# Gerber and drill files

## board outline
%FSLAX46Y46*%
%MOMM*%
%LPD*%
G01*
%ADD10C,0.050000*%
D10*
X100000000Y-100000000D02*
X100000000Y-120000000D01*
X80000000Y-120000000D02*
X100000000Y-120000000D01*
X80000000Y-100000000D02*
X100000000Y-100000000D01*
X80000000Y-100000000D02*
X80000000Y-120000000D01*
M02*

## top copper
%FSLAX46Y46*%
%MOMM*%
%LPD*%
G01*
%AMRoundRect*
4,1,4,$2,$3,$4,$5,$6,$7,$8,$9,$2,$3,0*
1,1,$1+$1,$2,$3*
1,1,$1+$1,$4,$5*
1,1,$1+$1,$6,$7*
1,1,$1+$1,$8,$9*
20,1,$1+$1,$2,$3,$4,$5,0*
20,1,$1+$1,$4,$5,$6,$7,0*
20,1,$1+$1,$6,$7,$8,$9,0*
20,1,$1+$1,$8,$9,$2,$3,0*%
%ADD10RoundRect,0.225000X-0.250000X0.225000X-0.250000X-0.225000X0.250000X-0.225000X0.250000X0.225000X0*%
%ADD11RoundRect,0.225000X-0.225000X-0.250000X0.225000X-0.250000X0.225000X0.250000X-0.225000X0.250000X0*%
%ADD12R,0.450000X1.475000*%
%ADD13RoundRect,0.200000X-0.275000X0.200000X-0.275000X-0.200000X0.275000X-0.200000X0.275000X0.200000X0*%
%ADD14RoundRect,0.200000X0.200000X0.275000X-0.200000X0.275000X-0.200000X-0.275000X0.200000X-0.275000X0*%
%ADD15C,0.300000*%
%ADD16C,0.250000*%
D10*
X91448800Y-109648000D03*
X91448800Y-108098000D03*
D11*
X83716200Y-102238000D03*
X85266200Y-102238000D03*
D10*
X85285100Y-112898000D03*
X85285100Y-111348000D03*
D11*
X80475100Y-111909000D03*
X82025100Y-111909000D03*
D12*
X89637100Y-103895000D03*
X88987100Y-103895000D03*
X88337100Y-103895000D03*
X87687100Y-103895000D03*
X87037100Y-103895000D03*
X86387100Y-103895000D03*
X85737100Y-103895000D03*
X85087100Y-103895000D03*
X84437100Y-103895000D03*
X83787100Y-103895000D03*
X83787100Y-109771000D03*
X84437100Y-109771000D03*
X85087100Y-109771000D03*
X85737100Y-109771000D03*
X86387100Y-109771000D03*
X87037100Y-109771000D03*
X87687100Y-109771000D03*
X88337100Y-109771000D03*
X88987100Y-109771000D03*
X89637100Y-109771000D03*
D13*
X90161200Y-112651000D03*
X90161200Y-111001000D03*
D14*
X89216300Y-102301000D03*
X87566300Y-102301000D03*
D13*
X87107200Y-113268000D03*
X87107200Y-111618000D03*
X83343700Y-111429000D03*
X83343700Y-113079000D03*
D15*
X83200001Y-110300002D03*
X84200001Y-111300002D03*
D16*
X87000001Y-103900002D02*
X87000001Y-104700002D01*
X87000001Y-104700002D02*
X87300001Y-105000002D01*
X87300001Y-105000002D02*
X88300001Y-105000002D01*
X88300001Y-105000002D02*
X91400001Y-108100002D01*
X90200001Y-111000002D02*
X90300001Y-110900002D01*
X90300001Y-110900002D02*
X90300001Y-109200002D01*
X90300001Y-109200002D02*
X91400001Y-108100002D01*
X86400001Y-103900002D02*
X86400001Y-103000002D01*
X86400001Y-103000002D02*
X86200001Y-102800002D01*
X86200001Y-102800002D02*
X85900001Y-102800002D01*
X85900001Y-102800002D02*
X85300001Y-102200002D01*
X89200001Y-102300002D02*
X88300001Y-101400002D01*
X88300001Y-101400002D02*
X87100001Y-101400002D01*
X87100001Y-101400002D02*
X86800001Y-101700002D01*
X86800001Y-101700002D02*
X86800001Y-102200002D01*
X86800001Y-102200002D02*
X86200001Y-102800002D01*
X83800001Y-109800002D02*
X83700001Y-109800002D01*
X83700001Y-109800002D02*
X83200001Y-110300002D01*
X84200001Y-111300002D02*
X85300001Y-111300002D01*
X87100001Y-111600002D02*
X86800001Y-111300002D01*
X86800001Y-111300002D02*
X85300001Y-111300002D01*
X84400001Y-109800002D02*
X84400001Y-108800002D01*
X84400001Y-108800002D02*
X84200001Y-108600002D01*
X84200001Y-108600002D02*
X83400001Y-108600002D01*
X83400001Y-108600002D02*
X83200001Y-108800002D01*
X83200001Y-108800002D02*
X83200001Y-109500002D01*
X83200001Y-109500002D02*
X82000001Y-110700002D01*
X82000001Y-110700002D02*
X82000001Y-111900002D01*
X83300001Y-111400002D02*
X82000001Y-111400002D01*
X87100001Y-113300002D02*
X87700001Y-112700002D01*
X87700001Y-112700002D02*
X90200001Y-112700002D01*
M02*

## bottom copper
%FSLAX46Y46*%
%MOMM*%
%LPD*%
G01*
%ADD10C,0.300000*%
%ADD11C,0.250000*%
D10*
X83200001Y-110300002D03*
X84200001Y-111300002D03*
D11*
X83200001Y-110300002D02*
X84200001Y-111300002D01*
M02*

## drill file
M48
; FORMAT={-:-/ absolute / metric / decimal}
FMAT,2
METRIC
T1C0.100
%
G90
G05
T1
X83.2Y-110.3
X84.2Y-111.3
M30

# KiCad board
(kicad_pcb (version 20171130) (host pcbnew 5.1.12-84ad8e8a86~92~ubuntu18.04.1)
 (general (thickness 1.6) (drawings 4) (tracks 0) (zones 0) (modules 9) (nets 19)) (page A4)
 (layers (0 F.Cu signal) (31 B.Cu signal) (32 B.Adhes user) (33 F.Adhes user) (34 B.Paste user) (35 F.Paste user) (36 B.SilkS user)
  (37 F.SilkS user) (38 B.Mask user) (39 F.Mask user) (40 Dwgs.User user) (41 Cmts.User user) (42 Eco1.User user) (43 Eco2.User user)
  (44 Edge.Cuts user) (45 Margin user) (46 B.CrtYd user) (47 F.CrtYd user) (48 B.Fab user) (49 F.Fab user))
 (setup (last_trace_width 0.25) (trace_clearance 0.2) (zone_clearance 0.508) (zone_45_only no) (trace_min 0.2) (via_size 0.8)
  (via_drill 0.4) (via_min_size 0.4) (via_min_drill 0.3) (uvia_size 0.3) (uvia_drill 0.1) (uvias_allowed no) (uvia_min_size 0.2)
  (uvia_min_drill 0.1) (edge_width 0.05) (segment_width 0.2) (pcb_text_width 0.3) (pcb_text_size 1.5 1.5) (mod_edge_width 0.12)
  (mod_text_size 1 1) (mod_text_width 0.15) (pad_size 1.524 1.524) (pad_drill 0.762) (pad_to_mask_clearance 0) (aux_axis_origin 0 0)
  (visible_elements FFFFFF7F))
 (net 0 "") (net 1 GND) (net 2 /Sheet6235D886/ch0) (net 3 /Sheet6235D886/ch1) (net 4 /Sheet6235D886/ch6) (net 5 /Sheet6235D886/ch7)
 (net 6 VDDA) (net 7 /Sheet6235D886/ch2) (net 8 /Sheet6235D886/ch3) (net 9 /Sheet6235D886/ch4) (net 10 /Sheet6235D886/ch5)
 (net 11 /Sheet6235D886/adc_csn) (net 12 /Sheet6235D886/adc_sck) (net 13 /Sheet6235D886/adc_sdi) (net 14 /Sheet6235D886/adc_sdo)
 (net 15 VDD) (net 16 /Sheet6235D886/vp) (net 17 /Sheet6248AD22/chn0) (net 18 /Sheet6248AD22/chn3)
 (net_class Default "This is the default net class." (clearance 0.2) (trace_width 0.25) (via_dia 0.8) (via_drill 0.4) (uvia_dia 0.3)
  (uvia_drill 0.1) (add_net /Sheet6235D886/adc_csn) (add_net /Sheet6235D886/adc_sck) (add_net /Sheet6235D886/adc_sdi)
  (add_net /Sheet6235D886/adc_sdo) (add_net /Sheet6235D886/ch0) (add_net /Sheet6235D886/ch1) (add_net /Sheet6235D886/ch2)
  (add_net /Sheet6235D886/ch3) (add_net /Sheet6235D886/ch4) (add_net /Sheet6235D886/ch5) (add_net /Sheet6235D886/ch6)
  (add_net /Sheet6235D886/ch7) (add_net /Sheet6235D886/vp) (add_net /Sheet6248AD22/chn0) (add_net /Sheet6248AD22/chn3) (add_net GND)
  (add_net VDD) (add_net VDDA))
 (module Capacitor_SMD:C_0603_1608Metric (layer F.Cu) (at 91.448800 108.873000 270.000000)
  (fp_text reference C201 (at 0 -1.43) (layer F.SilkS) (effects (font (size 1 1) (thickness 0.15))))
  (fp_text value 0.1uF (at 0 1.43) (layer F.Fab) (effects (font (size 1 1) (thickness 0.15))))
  (pad 2 smd roundrect (at 0.775 0 270.000000) (size 0.9 0.95) (layers F.Cu F.Mask F.Paste) (roundrect_rratio 0.25) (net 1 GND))
  (pad 1 smd roundrect (at -0.775 0 270.000000) (size 0.9 0.95) (layers F.Cu F.Mask F.Paste) (roundrect_rratio 0.25)
   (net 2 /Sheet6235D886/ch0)))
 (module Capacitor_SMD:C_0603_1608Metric (layer F.Cu) (at 84.491200 102.238000)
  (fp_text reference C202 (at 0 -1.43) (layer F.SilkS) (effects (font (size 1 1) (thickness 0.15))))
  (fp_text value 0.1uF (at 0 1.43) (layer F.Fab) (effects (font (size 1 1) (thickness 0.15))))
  (pad 1 smd roundrect (at -0.775 0) (size 0.9 0.95) (layers F.Cu F.Mask F.Paste) (roundrect_rratio 0.25) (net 1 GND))
  (pad 2 smd roundrect (at 0.775 0) (size 0.9 0.95) (layers F.Cu F.Mask F.Paste) (roundrect_rratio 0.25) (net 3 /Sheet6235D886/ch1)))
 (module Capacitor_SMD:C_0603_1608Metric (layer F.Cu) (at 85.285100 112.123000 270.000000)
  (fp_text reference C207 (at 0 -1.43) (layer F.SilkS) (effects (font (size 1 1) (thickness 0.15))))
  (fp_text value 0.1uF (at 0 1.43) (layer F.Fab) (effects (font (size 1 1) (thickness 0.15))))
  (pad 2 smd roundrect (at 0.775 0 270.000000) (size 0.9 0.95) (layers F.Cu F.Mask F.Paste) (roundrect_rratio 0.25) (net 1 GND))
  (pad 1 smd roundrect (at -0.775 0 270.000000) (size 0.9 0.95) (layers F.Cu F.Mask F.Paste) (roundrect_rratio 0.25)
   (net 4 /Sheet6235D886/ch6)))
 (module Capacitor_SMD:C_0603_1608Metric (layer F.Cu) (at 81.250100 111.909000)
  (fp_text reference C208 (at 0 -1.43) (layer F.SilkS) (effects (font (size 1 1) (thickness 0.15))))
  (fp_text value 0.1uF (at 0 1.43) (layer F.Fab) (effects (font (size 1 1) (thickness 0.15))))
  (pad 1 smd roundrect (at -0.775 0) (size 0.9 0.95) (layers F.Cu F.Mask F.Paste) (roundrect_rratio 0.25) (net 1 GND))
  (pad 2 smd roundrect (at 0.775 0) (size 0.9 0.95) (layers F.Cu F.Mask F.Paste) (roundrect_rratio 0.25) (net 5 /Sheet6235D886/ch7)))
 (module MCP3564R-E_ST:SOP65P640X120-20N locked (layer F.Cu) (at 86.712100 106.833000 270.000000)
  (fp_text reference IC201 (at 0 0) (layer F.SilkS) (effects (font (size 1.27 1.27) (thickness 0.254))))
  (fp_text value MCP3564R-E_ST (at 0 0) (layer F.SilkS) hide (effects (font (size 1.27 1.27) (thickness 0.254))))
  (pad 1 smd rect (at -2.938 -2.925) (size 0.45 1.475) (layers F.Cu F.Mask F.Paste) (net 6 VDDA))
  (pad 2 smd rect (at -2.938 -2.275) (size 0.45 1.475) (layers F.Cu F.Mask F.Paste) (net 1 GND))
  (pad 3 smd rect (at -2.938 -1.625) (size 0.45 1.475) (layers F.Cu F.Mask F.Paste) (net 1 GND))
  (pad 4 smd rect (at -2.938 -0.975) (size 0.45 1.475) (layers F.Cu F.Mask F.Paste))
  (pad 5 smd rect (at -2.938 -0.325) (size 0.45 1.475) (layers F.Cu F.Mask F.Paste) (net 2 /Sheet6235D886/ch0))
  (pad 6 smd rect (at -2.938 0.325) (size 0.45 1.475) (layers F.Cu F.Mask F.Paste) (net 3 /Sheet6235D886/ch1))
  (pad 7 smd rect (at -2.938 0.975) (size 0.45 1.475) (layers F.Cu F.Mask F.Paste) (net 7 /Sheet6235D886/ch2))
  (pad 8 smd rect (at -2.938 1.625) (size 0.45 1.475) (layers F.Cu F.Mask F.Paste) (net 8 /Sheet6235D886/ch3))
  (pad 9 smd rect (at -2.938 2.275) (size 0.45 1.475) (layers F.Cu F.Mask F.Paste) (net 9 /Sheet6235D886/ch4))
  (pad 10 smd rect (at -2.938 2.925) (size 0.45 1.475) (layers F.Cu F.Mask F.Paste) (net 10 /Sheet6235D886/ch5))
  (pad 11 smd rect (at 2.938 2.925) (size 0.45 1.475) (layers F.Cu F.Mask F.Paste) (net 4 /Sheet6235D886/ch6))
  (pad 12 smd rect (at 2.938 2.275) (size 0.45 1.475) (layers F.Cu F.Mask F.Paste) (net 5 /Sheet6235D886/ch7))
  (pad 13 smd rect (at 2.938 1.625) (size 0.45 1.475) (layers F.Cu F.Mask F.Paste) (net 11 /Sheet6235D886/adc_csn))
  (pad 14 smd rect (at 2.938 0.975) (size 0.45 1.475) (layers F.Cu F.Mask F.Paste) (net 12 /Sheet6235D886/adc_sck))
  (pad 15 smd rect (at 2.938 0.325) (size 0.45 1.475) (layers F.Cu F.Mask F.Paste) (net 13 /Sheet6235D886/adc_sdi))
  (pad 16 smd rect (at 2.938 -0.325) (size 0.45 1.475) (layers F.Cu F.Mask F.Paste) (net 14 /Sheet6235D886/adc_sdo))
  (pad 17 smd rect (at 2.938 -0.975) (size 0.45 1.475) (layers F.Cu F.Mask F.Paste))
  (pad 18 smd rect (at 2.938 -1.625) (size 0.45 1.475) (layers F.Cu F.Mask F.Paste))
  (pad 19 smd rect (at 2.938 -2.275) (size 0.45 1.475) (layers F.Cu F.Mask F.Paste) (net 1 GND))
  (pad 20 smd rect (at 2.938 -2.925) (size 0.45 1.475) (layers F.Cu F.Mask F.Paste) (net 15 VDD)))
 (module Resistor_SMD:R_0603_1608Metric (layer F.Cu) (at 90.161200 111.826000 270.000000)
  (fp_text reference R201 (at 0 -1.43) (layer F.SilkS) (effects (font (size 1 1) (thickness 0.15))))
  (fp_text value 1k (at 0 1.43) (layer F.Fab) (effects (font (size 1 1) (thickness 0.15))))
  (pad 2 smd roundrect (at 0.825 0 270.000000) (size 0.8 0.95) (layers F.Cu F.Mask F.Paste) (roundrect_rratio 0.25)
   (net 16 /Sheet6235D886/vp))
  (pad 1 smd roundrect (at -0.825 0 270.000000) (size 0.8 0.95) (layers F.Cu F.Mask F.Paste) (roundrect_rratio 0.25)
   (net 2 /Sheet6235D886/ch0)))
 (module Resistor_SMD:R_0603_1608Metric (layer F.Cu) (at 88.391300 102.301000 180.000000)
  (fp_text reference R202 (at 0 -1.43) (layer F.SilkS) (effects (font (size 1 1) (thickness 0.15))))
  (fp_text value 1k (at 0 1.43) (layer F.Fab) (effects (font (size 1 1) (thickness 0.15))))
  (pad 1 smd roundrect (at -0.825 0 180.000000) (size 0.8 0.95) (layers F.Cu F.Mask F.Paste) (roundrect_rratio 0.25)
   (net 3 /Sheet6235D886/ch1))
  (pad 2 smd roundrect (at 0.825 0 180.000000) (size 0.8 0.95) (layers F.Cu F.Mask F.Paste) (roundrect_rratio 0.25)
   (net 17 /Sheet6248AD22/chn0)))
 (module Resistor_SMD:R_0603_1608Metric (layer F.Cu) (at 87.107200 112.443000 270.000000)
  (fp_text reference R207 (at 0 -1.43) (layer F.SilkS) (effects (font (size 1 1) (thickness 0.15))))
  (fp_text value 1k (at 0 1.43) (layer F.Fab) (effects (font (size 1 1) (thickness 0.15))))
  (pad 2 smd roundrect (at 0.825 0 270.000000) (size 0.8 0.95) (layers F.Cu F.Mask F.Paste) (roundrect_rratio 0.25)
   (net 16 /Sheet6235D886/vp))
  (pad 1 smd roundrect (at -0.825 0 270.000000) (size 0.8 0.95) (layers F.Cu F.Mask F.Paste) (roundrect_rratio 0.25)
   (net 4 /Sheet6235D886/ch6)))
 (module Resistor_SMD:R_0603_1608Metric (layer F.Cu) (at 83.343700 112.254000 270.000000)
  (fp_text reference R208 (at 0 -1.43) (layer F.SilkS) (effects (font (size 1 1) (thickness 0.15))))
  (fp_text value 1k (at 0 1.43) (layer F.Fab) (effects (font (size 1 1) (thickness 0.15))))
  (pad 1 smd roundrect (at -0.825 0 270.000000) (size 0.8 0.95) (layers F.Cu F.Mask F.Paste) (roundrect_rratio 0.25)
   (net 5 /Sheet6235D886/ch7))
  (pad 2 smd roundrect (at 0.825 0 270.000000) (size 0.8 0.95) (layers F.Cu F.Mask F.Paste) (roundrect_rratio 0.25)
   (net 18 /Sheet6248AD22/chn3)))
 (gr_line (start 100 100) (end 100 120) (layer Edge.Cuts) (width 0.05))
 (gr_line (start 80 120) (end 100 120) (layer Edge.Cuts) (width 0.05))
 (gr_line (start 80 100) (end 100 100) (layer Edge.Cuts) (width 0.05))
 (gr_line (start 80 100) (end 80 120) (layer Edge.Cuts) (width 0.05))
 (segment (start 87.000001 103.900002) (end 87.000001 104.700002) (width 0.250000) (layer F.Cu) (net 2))
 (segment (start 87.000001 104.700002) (end 87.300001 105.000002) (width 0.250000) (layer F.Cu) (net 2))
 (segment (start 87.300001 105.000002) (end 88.300001 105.000002) (width 0.250000) (layer F.Cu) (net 2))
 (segment (start 88.300001 105.000002) (end 91.400001 108.100002) (width 0.250000) (layer F.Cu) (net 2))
 (segment (start 90.200001 111.000002) (end 90.300001 110.900002) (width 0.250000) (layer F.Cu) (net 2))
 (segment (start 90.300001 110.900002) (end 90.300001 109.200002) (width 0.250000) (layer F.Cu) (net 2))
 (segment (start 90.300001 109.200002) (end 91.400001 108.100002) (width 0.250000) (layer F.Cu) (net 2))
 (segment (start 86.400001 103.900002) (end 86.400001 103.000002) (width 0.250000) (layer F.Cu) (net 3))
 (segment (start 86.400001 103.000002) (end 86.200001 102.800002) (width 0.250000) (layer F.Cu) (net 3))
 (segment (start 86.200001 102.800002) (end 85.900001 102.800002) (width 0.250000) (layer F.Cu) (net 3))
 (segment (start 85.900001 102.800002) (end 85.300001 102.200002) (width 0.250000) (layer F.Cu) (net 3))
 (segment (start 89.200001 102.300002) (end 88.300001 101.400002) (width 0.250000) (layer F.Cu) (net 3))
 (segment (start 88.300001 101.400002) (end 87.100001 101.400002) (width 0.250000) (layer F.Cu) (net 3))
 (segment (start 87.100001 101.400002) (end 86.800001 101.700002) (width 0.250000) (layer F.Cu) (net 3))
 (segment (start 86.800001 101.700002) (end 86.800001 102.200002) (width 0.250000) (layer F.Cu) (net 3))
 (segment (start 86.800001 102.200002) (end 86.200001 102.800002) (width 0.250000) (layer F.Cu) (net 3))
 (segment (start 83.800001 109.800002) (end 83.700001 109.800002) (width 0.250000) (layer F.Cu) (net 4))
 (segment (start 83.700001 109.800002) (end 83.200001 110.300002) (width 0.250000) (layer F.Cu) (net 4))
 (segment (start 83.200001 110.300002) (end 84.200001 111.300002) (width 0.250000) (layer B.Cu) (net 4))
 (segment (start 84.200001 111.300002) (end 85.300001 111.300002) (width 0.250000) (layer F.Cu) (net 4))
 (segment (start 87.100001 111.600002) (end 86.800001 111.300002) (width 0.250000) (layer F.Cu) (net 4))
 (segment (start 86.800001 111.300002) (end 85.300001 111.300002) (width 0.250000) (layer F.Cu) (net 4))
 (via micro (at 83.200001 110.300002) (size 0.300000) (drill 0.100000) (layers F.Cu B.Cu) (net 4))
 (via micro (at 84.200001 111.300002) (size 0.300000) (drill 0.100000) (layers F.Cu B.Cu) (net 4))
 (segment (start 84.400001 109.800002) (end 84.400001 108.800002) (width 0.250000) (layer F.Cu) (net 5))
 (segment (start 84.400001 108.800002) (end 84.200001 108.600002) (width 0.250000) (layer F.Cu) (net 5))
 (segment (start 84.200001 108.600002) (end 83.400001 108.600002) (width 0.250000) (layer F.Cu) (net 5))
 (segment (start 83.400001 108.600002) (end 83.200001 108.800002) (width 0.250000) (layer F.Cu) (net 5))
 (segment (start 83.200001 108.800002) (end 83.200001 109.500002) (width 0.250000) (layer F.Cu) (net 5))
 (segment (start 83.200001 109.500002) (end 82.000001 110.700002) (width 0.250000) (layer F.Cu) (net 5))
 (segment (start 82.000001 110.700002) (end 82.000001 111.900002) (width 0.250000) (layer F.Cu) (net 5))
 (segment (start 83.300001 111.400002) (end 82.000001 111.400002) (width 0.250000) (layer F.Cu) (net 5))
 (segment (start 87.100001 113.300002) (end 87.700001 112.700002) (width 0.250000) (layer F.Cu) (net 16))
 (segment (start 87.700001 112.700002) (end 90.200001 112.700002) (width 0.250000) (layer F.Cu) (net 16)))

